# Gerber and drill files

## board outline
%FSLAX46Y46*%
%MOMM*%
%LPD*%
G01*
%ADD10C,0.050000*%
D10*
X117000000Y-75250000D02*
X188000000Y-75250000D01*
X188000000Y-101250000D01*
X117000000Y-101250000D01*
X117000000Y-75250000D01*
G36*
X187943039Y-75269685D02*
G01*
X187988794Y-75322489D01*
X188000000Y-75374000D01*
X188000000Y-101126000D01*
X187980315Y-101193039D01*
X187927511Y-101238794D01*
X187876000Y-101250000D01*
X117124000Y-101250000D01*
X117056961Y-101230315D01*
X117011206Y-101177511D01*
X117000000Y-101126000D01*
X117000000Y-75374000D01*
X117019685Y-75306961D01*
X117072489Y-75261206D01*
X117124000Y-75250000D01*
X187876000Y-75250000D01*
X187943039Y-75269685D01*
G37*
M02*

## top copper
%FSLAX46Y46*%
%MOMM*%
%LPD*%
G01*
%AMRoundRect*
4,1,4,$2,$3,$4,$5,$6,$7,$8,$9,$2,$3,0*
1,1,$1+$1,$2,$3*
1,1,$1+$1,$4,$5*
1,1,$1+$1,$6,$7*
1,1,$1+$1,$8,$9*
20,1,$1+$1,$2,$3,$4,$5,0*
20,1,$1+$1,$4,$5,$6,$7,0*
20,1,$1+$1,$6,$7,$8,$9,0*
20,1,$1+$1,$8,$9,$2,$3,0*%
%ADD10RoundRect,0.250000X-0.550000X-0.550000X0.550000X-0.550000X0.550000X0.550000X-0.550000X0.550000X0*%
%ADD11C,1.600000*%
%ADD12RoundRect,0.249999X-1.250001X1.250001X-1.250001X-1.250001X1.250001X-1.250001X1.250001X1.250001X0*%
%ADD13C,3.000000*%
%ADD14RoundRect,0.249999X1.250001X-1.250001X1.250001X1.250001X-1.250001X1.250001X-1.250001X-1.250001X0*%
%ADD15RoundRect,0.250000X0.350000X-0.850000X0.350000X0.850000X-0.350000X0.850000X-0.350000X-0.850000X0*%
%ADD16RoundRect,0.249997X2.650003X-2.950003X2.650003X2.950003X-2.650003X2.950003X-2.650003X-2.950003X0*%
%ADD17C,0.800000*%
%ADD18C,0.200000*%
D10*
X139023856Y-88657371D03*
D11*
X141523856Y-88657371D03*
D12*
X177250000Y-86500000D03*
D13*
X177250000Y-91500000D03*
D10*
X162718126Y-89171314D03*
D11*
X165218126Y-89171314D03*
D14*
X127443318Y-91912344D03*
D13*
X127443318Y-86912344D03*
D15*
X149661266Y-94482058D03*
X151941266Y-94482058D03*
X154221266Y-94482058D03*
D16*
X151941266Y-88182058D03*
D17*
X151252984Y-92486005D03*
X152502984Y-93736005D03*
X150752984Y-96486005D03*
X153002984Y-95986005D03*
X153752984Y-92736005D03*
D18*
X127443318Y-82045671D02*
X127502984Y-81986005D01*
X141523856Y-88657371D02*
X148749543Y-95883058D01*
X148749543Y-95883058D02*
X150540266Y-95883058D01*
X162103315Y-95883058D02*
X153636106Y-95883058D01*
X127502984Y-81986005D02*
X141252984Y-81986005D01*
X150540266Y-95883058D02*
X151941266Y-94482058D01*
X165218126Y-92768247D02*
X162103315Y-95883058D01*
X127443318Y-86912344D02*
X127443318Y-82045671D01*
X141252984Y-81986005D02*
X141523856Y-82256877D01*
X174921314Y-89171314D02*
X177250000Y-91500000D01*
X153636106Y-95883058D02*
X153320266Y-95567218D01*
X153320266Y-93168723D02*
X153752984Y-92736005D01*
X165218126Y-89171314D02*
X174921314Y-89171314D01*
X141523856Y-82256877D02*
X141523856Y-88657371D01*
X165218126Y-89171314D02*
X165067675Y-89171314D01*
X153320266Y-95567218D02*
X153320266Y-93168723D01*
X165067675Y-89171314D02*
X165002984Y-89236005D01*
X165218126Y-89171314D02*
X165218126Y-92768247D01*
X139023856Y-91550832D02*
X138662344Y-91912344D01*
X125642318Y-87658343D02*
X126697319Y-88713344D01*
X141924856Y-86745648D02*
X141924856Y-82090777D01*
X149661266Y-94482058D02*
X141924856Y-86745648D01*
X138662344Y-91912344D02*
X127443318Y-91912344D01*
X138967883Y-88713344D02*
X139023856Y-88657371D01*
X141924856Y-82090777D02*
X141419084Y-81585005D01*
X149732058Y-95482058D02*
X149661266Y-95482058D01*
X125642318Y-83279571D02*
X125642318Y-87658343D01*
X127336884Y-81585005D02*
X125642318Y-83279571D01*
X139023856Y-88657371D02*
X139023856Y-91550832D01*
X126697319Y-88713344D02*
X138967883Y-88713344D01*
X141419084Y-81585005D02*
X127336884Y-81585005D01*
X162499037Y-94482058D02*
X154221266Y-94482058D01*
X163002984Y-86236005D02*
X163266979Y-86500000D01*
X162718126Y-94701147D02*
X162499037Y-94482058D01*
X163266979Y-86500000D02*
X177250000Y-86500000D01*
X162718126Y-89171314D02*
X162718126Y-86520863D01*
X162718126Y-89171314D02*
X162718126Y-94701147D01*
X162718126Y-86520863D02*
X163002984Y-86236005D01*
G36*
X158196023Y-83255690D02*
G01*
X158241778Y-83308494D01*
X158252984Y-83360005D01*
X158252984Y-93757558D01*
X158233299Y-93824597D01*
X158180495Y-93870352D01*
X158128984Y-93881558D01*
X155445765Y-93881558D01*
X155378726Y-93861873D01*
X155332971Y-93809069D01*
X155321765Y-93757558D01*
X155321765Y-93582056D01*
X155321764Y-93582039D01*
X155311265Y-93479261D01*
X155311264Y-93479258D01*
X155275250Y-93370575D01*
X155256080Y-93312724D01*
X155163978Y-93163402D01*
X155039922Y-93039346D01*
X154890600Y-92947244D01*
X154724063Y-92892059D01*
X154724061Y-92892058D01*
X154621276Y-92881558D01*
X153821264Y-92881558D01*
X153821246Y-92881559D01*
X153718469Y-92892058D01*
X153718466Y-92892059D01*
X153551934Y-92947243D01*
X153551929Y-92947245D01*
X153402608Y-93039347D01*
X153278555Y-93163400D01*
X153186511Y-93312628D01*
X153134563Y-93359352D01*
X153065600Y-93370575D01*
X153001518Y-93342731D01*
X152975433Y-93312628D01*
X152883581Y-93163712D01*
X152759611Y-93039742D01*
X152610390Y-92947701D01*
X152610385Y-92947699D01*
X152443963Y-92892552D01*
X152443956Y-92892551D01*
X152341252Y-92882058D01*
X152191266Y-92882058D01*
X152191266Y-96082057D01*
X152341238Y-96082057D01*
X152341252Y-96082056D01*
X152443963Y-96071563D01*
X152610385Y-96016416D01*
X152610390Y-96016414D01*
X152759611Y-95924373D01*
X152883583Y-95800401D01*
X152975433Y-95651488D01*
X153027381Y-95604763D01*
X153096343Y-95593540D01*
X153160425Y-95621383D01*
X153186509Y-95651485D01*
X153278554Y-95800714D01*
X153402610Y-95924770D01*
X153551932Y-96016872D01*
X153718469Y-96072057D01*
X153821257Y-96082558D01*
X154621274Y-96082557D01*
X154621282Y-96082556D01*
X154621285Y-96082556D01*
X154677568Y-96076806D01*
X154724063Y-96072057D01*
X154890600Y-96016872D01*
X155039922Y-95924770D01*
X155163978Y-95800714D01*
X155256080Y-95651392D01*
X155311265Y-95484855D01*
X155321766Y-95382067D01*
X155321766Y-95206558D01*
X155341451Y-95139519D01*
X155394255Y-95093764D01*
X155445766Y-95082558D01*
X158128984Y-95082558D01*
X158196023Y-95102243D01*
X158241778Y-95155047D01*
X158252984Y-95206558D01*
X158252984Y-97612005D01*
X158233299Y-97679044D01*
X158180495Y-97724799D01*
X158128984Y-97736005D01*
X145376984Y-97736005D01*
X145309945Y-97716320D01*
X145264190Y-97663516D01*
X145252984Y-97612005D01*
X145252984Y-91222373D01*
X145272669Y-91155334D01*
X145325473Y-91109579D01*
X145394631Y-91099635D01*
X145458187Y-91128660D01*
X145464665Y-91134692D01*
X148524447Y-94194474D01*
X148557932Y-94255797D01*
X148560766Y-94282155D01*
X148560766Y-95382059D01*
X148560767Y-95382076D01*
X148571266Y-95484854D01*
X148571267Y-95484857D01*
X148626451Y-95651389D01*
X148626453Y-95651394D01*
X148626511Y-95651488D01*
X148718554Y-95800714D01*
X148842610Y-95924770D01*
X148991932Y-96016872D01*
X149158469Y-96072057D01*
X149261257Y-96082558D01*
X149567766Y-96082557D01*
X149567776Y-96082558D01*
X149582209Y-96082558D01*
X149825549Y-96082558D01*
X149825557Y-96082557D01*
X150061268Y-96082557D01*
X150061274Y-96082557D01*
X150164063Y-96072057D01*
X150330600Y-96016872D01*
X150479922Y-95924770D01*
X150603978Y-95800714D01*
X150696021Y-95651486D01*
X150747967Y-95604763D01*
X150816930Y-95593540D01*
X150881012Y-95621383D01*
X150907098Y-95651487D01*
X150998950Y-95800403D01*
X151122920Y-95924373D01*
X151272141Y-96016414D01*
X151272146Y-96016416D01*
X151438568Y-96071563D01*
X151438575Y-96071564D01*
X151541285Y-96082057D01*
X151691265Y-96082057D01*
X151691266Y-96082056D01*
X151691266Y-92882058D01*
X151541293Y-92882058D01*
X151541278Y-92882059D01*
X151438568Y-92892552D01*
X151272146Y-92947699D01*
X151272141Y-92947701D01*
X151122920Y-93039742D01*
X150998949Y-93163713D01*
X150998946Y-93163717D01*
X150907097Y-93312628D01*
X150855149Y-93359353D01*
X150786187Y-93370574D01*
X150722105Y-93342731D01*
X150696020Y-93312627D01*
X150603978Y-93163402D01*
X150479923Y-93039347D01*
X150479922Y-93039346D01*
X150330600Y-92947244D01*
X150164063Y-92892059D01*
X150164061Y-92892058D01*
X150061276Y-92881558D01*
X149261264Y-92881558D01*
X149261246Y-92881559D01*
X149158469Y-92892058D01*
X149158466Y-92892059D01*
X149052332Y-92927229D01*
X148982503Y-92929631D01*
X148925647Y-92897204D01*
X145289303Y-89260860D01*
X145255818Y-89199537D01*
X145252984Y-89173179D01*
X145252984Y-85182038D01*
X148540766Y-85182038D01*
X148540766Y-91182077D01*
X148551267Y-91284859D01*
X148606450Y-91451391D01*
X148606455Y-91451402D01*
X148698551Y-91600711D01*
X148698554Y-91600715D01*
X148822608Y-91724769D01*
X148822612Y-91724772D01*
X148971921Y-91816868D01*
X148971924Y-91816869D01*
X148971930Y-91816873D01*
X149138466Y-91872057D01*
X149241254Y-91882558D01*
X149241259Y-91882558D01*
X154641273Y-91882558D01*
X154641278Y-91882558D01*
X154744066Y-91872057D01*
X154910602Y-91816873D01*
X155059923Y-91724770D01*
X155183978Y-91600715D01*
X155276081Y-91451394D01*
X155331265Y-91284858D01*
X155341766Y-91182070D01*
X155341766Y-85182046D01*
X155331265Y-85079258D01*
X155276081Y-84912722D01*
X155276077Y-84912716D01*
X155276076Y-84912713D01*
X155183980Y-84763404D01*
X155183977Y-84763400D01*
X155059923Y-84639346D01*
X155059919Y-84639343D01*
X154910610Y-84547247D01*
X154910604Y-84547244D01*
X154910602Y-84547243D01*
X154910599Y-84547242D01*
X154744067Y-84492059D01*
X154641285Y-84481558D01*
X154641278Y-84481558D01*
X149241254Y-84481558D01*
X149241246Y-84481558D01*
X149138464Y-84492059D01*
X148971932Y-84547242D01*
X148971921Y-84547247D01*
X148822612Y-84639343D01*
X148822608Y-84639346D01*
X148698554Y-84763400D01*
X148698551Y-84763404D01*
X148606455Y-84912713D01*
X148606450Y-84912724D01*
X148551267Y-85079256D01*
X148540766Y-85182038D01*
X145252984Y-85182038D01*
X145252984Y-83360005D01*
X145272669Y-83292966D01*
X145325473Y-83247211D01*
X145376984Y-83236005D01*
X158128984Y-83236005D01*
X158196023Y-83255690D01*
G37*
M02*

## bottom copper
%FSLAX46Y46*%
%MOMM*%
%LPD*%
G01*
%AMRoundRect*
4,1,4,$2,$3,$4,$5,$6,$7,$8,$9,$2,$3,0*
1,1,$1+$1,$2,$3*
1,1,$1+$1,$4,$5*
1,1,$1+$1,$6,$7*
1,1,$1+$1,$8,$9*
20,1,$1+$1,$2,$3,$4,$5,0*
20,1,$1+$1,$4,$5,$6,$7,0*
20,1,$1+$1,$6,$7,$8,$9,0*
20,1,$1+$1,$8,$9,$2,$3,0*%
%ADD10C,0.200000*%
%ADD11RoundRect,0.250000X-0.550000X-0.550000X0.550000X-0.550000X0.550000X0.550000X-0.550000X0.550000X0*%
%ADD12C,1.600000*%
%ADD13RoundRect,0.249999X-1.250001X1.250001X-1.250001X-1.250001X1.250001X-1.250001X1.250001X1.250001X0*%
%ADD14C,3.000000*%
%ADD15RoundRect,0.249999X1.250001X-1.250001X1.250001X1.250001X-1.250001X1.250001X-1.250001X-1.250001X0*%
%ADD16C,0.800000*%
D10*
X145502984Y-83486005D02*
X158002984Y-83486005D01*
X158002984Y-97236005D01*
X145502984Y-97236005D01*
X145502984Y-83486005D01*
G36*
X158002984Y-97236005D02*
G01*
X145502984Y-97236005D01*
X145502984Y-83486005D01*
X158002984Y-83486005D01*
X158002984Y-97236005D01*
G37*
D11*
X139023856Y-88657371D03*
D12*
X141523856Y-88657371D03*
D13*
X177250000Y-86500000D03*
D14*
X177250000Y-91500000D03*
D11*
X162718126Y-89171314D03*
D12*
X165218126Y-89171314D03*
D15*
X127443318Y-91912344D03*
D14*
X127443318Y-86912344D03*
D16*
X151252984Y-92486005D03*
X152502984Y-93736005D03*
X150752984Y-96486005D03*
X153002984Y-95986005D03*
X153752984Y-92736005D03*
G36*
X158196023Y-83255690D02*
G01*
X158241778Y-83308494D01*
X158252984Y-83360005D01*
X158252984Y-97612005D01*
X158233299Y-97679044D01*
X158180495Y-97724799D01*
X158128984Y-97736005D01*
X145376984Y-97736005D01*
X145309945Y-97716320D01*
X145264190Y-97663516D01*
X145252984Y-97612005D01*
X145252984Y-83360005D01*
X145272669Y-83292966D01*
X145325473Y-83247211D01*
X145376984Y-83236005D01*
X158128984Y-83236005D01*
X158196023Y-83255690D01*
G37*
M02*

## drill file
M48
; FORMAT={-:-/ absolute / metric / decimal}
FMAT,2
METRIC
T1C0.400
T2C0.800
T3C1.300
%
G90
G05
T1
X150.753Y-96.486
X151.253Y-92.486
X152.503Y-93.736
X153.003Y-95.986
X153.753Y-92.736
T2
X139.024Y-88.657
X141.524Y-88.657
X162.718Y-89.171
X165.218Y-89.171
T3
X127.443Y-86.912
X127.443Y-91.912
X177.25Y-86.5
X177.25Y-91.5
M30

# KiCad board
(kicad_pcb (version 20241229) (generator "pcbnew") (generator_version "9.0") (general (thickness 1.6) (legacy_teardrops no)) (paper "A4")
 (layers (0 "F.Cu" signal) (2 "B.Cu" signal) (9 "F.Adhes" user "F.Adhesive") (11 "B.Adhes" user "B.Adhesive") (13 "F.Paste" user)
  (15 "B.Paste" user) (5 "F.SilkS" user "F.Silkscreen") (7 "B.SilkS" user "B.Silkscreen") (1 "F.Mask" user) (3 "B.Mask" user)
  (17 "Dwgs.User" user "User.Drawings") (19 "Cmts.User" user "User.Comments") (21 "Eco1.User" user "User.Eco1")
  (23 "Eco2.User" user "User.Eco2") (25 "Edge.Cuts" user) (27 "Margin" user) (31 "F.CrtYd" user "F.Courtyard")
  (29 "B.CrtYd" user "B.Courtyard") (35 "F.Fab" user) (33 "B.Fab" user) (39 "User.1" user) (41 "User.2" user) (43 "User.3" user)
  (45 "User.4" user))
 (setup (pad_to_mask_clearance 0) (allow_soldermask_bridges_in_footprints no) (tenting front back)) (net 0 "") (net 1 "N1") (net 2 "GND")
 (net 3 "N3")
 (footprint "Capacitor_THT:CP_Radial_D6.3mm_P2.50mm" (layer "F.Cu") (at 139.023856 88.657371)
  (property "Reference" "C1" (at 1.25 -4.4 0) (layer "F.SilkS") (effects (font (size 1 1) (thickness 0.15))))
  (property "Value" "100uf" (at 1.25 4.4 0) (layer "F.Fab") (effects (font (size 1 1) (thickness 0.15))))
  (pad "1" thru_hole roundrect (at 0 0) (size 1.6 1.6) (drill 0.8) (layers "*.Cu" "*.Mask") (remove_unused_layers no)
   (roundrect_rratio 0.15625) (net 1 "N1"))
  (pad "2" thru_hole circle (at 2.5 0) (size 1.6 1.6) (drill 0.8) (layers "*.Cu" "*.Mask") (remove_unused_layers no) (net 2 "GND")))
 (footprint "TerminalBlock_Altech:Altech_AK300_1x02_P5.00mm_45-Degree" (layer "F.Cu") (at 177.25 86.5 -90)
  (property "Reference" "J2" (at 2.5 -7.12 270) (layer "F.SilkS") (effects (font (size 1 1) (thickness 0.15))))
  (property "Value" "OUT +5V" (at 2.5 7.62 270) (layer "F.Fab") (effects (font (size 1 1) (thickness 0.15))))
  (pad "1" thru_hole roundrect (at 0 0 270) (size 3 3) (drill 1.3) (layers "*.Cu" "*.Mask") (remove_unused_layers no)
   (roundrect_rratio 0.083333) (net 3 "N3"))
  (pad "2" thru_hole circle (at 5 0 270) (size 3 3) (drill 1.3) (layers "*.Cu" "*.Mask") (remove_unused_layers no) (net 2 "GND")))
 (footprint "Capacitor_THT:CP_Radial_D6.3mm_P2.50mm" (layer "F.Cu") (at 162.718126 89.171314)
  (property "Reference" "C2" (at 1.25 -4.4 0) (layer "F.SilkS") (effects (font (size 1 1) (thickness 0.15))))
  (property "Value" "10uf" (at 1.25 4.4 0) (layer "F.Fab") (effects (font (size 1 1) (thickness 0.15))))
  (pad "1" thru_hole roundrect (at 0 0) (size 1.6 1.6) (drill 0.8) (layers "*.Cu" "*.Mask") (remove_unused_layers no)
   (roundrect_rratio 0.15625) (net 3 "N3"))
  (pad "2" thru_hole circle (at 2.5 0) (size 1.6 1.6) (drill 0.8) (layers "*.Cu" "*.Mask") (remove_unused_layers no) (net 2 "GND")))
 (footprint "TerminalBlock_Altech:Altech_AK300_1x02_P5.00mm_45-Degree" (layer "F.Cu") (at 127.443318 91.912344 90)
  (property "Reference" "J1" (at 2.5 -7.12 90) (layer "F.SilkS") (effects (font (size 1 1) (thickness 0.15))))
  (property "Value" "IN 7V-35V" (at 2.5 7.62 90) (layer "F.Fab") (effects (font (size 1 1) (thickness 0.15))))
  (pad "1" thru_hole roundrect (at 0 0 90) (size 3 3) (drill 1.3) (layers "*.Cu" "*.Mask") (remove_unused_layers no)
   (roundrect_rratio 0.083333) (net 1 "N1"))
  (pad "2" thru_hole circle (at 5 0 90) (size 3 3) (drill 1.3) (layers "*.Cu" "*.Mask") (remove_unused_layers no) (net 2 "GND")))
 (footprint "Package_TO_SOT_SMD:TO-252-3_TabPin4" (layer "F.Cu") (at 151.941266 89.442058 90)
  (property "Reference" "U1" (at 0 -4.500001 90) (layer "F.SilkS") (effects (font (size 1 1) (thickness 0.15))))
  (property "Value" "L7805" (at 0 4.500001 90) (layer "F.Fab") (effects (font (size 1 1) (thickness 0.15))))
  (pad "" smd roundrect (at -0.415 -1.525 90) (size 3.05 2.75) (layers "F.Paste") (roundrect_rratio 0.090909))
  (pad "" smd roundrect (at -0.415 1.525 90) (size 3.05 2.75) (layers "F.Paste") (roundrect_rratio 0.090909))
  (pad "" smd roundrect (at 2.935 -1.525 90) (size 3.05 2.75) (layers "F.Paste") (roundrect_rratio 0.090909))
  (pad "" smd roundrect (at 2.935 1.525 90) (size 3.05 2.75) (layers "F.Paste") (roundrect_rratio 0.090909))
  (pad "1" smd roundrect (at -5.04 -2.28 90) (size 2.2 1.2) (layers "F.Cu" "F.Mask" "F.Paste") (roundrect_rratio 0.208333) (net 1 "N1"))
  (pad "2" smd roundrect (at -5.04 0 90) (size 2.2 1.2) (layers "F.Cu" "F.Mask" "F.Paste") (roundrect_rratio 0.208333) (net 2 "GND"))
  (pad "3" smd roundrect (at -5.04 2.28 90) (size 2.2 1.2) (layers "F.Cu" "F.Mask" "F.Paste") (roundrect_rratio 0.208333) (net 3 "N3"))
  (pad "4" smd roundrect (at 1.26 0 90) (size 6.4 5.8) (layers "F.Cu" "F.Mask") (roundrect_rratio 0.043103)))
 (gr_poly
  (pts (xy 145.502984 83.486005) (xy 158.002984 83.486005) (xy 158.002984 97.236005) (xy 145.502984 97.236005))
  (stroke (width 0.2) (type solid)) (fill yes) (layer "B.Cu") (net 2))
 (gr_rect (start 117 75.25) (end 188 101.25) (stroke (width 0.05) (type default)) (fill no) (layer "Edge.Cuts"))
 (segment (start 127.443318 82.045671) (end 127.502984 81.986005) (width 0.2) (layer "F.Cu") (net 2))
 (segment (start 141.523856 88.657371) (end 148.749543 95.883058) (width 0.2) (layer "F.Cu") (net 2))
 (segment (start 148.749543 95.883058) (end 150.540266 95.883058) (width 0.2) (layer "F.Cu") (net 2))
 (segment (start 162.103315 95.883058) (end 153.636106 95.883058) (width 0.2) (layer "F.Cu") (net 2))
 (segment (start 127.502984 81.986005) (end 141.252984 81.986005) (width 0.2) (layer "F.Cu") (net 2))
 (segment (start 150.540266 95.883058) (end 151.941266 94.482058) (width 0.2) (layer "F.Cu") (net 2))
 (segment (start 165.218126 92.768247) (end 162.103315 95.883058) (width 0.2) (layer "F.Cu") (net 2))
 (segment (start 127.443318 86.912344) (end 127.443318 82.045671) (width 0.2) (layer "F.Cu") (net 2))
 (segment (start 141.252984 81.986005) (end 141.523856 82.256877) (width 0.2) (layer "F.Cu") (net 2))
 (segment (start 174.921314 89.171314) (end 177.25 91.5) (width 0.2) (layer "F.Cu") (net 2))
 (segment (start 153.636106 95.883058) (end 153.320266 95.567218) (width 0.2) (layer "F.Cu") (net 2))
 (segment (start 153.320266 93.168723) (end 153.752984 92.736005) (width 0.2) (layer "F.Cu") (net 2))
 (segment (start 165.218126 89.171314) (end 174.921314 89.171314) (width 0.2) (layer "F.Cu") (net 2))
 (segment (start 141.523856 82.256877) (end 141.523856 88.657371) (width 0.2) (layer "F.Cu") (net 2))
 (segment (start 165.218126 89.171314) (end 165.067675 89.171314) (width 0.2) (layer "F.Cu") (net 2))
 (segment (start 153.320266 95.567218) (end 153.320266 93.168723) (width 0.2) (layer "F.Cu") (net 2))
 (segment (start 165.067675 89.171314) (end 165.002984 89.236005) (width 0.2) (layer "F.Cu") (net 2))
 (segment (start 165.218126 89.171314) (end 165.218126 92.768247) (width 0.2) (layer "F.Cu") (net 2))
 (via (at 151.252984 92.486005) (size 0.8) (drill 0.4) (layers "F.Cu" "B.Cu") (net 2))
 (via (at 152.502984 93.736005) (size 0.8) (drill 0.4) (layers "F.Cu" "B.Cu") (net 2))
 (via (at 150.752984 96.486005) (size 0.8) (drill 0.4) (layers "F.Cu" "B.Cu") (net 2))
 (via (at 153.002984 95.986005) (size 0.8) (drill 0.4) (layers "F.Cu" "B.Cu") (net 2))
 (via (at 153.752984 92.736005) (size 0.8) (drill 0.4) (layers "F.Cu" "B.Cu") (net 2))
 (segment (start 139.023856 91.550832) (end 138.662344 91.912344) (width 0.2) (layer "F.Cu") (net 1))
 (segment (start 125.642318 87.658343) (end 126.697319 88.713344) (width 0.2) (layer "F.Cu") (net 1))
 (segment (start 141.924856 86.745648) (end 141.924856 82.090777) (width 0.2) (layer "F.Cu") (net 1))
 (segment (start 149.661266 94.482058) (end 141.924856 86.745648) (width 0.2) (layer "F.Cu") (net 1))
 (segment (start 138.662344 91.912344) (end 127.443318 91.912344) (width 0.2) (layer "F.Cu") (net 1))
 (segment (start 138.967883 88.713344) (end 139.023856 88.657371) (width 0.2) (layer "F.Cu") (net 1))
 (segment (start 141.924856 82.090777) (end 141.419084 81.585005) (width 0.2) (layer "F.Cu") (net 1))
 (segment (start 149.732058 95.482058) (end 149.661266 95.482058) (width 0.2) (layer "F.Cu") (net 1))
 (segment (start 125.642318 83.279571) (end 125.642318 87.658343) (width 0.2) (layer "F.Cu") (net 1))
 (segment (start 127.336884 81.585005) (end 125.642318 83.279571) (width 0.2) (layer "F.Cu") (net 1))
 (segment (start 139.023856 88.657371) (end 139.023856 91.550832) (width 0.2) (layer "F.Cu") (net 1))
 (segment (start 126.697319 88.713344) (end 138.967883 88.713344) (width 0.2) (layer "F.Cu") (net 1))
 (segment (start 141.419084 81.585005) (end 127.336884 81.585005) (width 0.2) (layer "F.Cu") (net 1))
 (segment (start 162.499037 94.482058) (end 154.221266 94.482058) (width 0.2) (layer "F.Cu") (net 3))
 (segment (start 163.002984 86.236005) (end 163.266979 86.5) (width 0.2) (layer "F.Cu") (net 3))
 (segment (start 162.718126 94.701147) (end 162.499037 94.482058) (width 0.2) (layer "F.Cu") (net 3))
 (segment (start 163.266979 86.5) (end 177.25 86.5) (width 0.2) (layer "F.Cu") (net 3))
 (segment (start 162.718126 89.171314) (end 162.718126 86.520863) (width 0.2) (layer "F.Cu") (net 3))
 (segment (start 162.718126 89.171314) (end 162.718126 94.701147) (width 0.2) (layer "F.Cu") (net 3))
 (segment (start 162.718126 86.520863) (end 163.002984 86.236005) (width 0.2) (layer "F.Cu") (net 3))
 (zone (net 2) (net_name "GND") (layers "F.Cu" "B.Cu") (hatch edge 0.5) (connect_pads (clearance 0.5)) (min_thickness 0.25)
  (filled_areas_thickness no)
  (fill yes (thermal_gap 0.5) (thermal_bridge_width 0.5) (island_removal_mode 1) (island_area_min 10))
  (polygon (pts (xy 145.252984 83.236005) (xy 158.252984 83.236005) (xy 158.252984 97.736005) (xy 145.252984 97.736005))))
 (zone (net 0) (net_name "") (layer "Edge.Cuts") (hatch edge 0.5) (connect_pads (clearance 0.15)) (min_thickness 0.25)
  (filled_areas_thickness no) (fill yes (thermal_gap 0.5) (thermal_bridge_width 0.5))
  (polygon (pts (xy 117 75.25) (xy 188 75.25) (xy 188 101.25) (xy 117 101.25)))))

